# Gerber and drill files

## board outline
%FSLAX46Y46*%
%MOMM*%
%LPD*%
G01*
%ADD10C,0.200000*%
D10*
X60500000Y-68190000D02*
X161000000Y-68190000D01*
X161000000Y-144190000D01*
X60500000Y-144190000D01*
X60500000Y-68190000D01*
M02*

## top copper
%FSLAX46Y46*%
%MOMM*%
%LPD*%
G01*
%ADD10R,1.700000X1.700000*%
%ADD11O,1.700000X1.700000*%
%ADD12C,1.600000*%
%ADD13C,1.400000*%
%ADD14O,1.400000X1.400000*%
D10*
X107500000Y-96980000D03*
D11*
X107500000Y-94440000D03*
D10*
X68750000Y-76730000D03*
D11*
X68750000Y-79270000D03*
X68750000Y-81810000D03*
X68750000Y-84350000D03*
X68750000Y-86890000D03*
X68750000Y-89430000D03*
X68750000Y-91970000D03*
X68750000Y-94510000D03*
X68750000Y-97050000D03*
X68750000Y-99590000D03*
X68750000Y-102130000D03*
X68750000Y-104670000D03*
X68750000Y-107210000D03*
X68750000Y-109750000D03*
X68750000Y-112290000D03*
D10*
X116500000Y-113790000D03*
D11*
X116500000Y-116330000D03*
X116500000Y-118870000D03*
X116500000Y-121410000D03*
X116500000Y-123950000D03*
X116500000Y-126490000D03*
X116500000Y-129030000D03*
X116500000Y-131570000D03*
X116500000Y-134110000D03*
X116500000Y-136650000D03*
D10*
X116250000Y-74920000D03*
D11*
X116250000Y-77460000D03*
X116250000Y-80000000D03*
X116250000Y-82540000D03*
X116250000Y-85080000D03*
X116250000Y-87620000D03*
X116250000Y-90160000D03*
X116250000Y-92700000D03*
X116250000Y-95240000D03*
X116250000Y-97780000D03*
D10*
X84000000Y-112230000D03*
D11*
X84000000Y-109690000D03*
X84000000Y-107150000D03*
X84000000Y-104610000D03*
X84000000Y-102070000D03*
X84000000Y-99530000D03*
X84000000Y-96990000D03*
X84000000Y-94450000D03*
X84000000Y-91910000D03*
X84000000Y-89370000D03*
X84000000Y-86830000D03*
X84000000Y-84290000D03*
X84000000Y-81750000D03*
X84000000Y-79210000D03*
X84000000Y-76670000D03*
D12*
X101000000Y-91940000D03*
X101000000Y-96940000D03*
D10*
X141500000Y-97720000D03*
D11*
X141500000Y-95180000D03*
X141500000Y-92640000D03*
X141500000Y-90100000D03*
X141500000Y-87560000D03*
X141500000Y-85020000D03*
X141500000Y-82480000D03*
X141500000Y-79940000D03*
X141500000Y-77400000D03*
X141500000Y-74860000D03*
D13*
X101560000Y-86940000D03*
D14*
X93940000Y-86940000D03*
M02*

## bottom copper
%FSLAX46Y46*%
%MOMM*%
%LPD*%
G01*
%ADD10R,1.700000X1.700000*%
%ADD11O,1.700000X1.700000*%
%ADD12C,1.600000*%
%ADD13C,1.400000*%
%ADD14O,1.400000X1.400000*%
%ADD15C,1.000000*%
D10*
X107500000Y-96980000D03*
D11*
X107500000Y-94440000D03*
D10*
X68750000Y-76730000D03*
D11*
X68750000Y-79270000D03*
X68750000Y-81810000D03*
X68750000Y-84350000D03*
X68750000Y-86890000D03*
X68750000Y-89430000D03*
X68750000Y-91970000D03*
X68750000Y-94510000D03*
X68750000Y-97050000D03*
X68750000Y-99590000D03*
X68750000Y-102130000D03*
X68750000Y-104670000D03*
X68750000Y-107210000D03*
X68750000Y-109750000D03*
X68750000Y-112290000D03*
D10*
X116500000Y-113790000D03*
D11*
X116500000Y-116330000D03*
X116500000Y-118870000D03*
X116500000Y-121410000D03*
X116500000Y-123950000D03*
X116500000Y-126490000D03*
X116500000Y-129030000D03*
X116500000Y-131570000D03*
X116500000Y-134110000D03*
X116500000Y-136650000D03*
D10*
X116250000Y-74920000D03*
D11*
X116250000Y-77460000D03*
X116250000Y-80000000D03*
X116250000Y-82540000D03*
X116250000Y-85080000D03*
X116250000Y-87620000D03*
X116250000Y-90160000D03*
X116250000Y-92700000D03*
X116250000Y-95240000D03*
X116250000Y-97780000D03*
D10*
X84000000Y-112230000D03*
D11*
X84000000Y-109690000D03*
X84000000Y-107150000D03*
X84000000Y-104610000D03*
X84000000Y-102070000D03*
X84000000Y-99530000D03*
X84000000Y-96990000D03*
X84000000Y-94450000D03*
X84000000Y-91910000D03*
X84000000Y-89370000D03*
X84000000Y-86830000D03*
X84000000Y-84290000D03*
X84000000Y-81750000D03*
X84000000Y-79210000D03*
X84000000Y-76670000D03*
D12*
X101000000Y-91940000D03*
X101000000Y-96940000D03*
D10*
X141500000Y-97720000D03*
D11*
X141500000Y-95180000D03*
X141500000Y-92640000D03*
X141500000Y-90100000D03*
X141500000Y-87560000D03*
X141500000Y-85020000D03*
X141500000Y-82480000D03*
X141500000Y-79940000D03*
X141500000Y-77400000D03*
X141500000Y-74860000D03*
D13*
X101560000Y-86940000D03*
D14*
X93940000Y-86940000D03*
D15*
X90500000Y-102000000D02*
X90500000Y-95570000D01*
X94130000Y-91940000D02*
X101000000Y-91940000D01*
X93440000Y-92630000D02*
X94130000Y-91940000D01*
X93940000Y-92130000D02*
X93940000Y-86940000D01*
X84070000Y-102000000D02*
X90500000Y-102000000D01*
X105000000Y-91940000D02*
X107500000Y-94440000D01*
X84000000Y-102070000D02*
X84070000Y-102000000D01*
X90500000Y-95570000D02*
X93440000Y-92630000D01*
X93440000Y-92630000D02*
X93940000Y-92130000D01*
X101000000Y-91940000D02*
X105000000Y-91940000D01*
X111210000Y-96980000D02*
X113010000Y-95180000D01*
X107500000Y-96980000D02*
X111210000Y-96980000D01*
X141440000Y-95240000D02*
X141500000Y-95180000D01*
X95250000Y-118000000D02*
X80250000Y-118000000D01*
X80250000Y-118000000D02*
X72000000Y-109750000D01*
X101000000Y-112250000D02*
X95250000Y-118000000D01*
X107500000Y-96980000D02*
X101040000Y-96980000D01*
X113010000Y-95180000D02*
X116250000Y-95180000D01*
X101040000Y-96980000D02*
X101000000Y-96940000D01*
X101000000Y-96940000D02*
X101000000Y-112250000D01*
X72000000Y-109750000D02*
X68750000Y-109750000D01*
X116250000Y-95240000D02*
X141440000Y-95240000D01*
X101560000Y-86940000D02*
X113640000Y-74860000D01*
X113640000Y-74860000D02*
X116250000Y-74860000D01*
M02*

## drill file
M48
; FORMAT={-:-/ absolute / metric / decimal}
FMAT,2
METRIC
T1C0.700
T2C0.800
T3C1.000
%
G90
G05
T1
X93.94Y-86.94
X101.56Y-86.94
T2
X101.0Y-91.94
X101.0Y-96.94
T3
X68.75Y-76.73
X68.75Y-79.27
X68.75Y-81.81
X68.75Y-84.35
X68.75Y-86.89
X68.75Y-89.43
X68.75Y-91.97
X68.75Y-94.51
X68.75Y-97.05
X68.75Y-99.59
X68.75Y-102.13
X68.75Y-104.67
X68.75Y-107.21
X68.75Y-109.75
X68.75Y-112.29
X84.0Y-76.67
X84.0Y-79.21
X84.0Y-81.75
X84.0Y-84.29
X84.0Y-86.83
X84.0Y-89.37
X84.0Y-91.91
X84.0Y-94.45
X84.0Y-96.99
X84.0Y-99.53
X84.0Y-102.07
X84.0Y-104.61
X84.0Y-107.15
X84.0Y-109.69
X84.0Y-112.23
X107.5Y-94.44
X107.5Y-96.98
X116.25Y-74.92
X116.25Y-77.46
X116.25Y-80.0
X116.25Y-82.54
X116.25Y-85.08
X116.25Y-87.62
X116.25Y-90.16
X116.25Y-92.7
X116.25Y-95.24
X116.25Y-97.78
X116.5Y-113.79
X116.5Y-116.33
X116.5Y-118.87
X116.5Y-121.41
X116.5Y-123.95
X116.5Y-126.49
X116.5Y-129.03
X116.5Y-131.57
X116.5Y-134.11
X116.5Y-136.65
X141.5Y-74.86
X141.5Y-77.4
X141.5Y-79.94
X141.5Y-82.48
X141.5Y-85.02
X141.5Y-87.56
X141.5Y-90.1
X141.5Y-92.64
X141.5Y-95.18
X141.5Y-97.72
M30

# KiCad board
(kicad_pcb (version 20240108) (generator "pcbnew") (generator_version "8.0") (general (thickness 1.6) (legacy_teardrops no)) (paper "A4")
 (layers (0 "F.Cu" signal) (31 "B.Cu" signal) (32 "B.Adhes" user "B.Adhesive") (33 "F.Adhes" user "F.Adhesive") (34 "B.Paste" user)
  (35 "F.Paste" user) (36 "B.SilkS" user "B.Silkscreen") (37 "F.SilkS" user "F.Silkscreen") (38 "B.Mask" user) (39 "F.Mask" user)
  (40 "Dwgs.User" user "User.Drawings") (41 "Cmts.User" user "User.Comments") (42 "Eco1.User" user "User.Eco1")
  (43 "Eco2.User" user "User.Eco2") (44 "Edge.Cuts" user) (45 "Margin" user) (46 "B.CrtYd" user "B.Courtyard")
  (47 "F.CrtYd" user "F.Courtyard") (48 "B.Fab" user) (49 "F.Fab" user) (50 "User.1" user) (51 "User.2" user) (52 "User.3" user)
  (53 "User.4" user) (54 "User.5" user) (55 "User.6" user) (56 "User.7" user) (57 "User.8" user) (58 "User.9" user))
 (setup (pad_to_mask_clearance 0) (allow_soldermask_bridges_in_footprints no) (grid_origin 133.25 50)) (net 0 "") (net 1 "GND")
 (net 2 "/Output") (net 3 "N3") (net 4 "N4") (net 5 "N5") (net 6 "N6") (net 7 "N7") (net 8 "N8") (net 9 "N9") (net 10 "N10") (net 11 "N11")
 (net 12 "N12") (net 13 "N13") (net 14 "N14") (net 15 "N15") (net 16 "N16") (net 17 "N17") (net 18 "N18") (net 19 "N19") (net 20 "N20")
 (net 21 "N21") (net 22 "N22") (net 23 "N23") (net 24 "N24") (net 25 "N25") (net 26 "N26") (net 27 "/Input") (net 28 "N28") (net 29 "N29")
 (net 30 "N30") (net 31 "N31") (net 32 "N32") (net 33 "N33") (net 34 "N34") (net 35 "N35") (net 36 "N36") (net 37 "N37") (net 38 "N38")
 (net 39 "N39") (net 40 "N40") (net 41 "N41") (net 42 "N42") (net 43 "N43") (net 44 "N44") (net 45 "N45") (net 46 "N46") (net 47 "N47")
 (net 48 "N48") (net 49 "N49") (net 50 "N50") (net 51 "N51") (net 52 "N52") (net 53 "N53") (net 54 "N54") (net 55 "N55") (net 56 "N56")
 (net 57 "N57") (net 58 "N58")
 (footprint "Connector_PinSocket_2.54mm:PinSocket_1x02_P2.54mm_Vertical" (layer "F.Cu") (at 107.5 96.98 180)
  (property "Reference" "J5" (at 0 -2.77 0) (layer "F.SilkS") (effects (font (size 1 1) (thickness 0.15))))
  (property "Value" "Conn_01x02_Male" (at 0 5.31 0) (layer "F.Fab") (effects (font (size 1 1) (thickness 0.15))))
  (pad "1" thru_hole rect (at 0 0 180) (size 1.7 1.7) (drill 1) (layers "*.Cu" "*.Mask") (remove_unused_layers no) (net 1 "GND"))
  (pad "2" thru_hole oval (at 0 2.54 180) (size 1.7 1.7) (drill 1) (layers "*.Cu" "*.Mask") (remove_unused_layers no) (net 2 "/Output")))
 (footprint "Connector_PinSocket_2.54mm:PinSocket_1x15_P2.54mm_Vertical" (layer "F.Cu") (at 68.75 76.73)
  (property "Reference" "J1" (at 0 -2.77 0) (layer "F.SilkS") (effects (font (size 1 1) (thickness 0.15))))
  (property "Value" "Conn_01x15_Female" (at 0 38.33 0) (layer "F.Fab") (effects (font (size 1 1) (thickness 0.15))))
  (pad "1" thru_hole rect (at 0 0) (size 1.7 1.7) (drill 1) (layers "*.Cu" "*.Mask") (remove_unused_layers no) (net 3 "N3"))
  (pad "2" thru_hole oval (at 0 2.54) (size 1.7 1.7) (drill 1) (layers "*.Cu" "*.Mask") (remove_unused_layers no) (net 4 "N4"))
  (pad "3" thru_hole oval (at 0 5.08) (size 1.7 1.7) (drill 1) (layers "*.Cu" "*.Mask") (remove_unused_layers no) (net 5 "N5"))
  (pad "4" thru_hole oval (at 0 7.62) (size 1.7 1.7) (drill 1) (layers "*.Cu" "*.Mask") (remove_unused_layers no) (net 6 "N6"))
  (pad "5" thru_hole oval (at 0 10.16) (size 1.7 1.7) (drill 1) (layers "*.Cu" "*.Mask") (remove_unused_layers no) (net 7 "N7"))
  (pad "6" thru_hole oval (at 0 12.7) (size 1.7 1.7) (drill 1) (layers "*.Cu" "*.Mask") (remove_unused_layers no) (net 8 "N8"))
  (pad "7" thru_hole oval (at 0 15.24) (size 1.7 1.7) (drill 1) (layers "*.Cu" "*.Mask") (remove_unused_layers no) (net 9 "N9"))
  (pad "8" thru_hole oval (at 0 17.78) (size 1.7 1.7) (drill 1) (layers "*.Cu" "*.Mask") (remove_unused_layers no) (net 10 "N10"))
  (pad "9" thru_hole oval (at 0 20.32) (size 1.7 1.7) (drill 1) (layers "*.Cu" "*.Mask") (remove_unused_layers no) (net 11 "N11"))
  (pad "10" thru_hole oval (at 0 22.86) (size 1.7 1.7) (drill 1) (layers "*.Cu" "*.Mask") (remove_unused_layers no) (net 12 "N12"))
  (pad "11" thru_hole oval (at 0 25.4) (size 1.7 1.7) (drill 1) (layers "*.Cu" "*.Mask") (remove_unused_layers no) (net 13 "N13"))
  (pad "12" thru_hole oval (at 0 27.94) (size 1.7 1.7) (drill 1) (layers "*.Cu" "*.Mask") (remove_unused_layers no) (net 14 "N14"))
  (pad "13" thru_hole oval (at 0 30.48) (size 1.7 1.7) (drill 1) (layers "*.Cu" "*.Mask") (remove_unused_layers no) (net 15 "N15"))
  (pad "14" thru_hole oval (at 0 33.02) (size 1.7 1.7) (drill 1) (layers "*.Cu" "*.Mask") (remove_unused_layers no) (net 1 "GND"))
  (pad "15" thru_hole oval (at 0 35.56) (size 1.7 1.7) (drill 1) (layers "*.Cu" "*.Mask") (remove_unused_layers no) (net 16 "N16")))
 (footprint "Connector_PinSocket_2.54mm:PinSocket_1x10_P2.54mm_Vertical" (layer "F.Cu") (at 116.5 113.79)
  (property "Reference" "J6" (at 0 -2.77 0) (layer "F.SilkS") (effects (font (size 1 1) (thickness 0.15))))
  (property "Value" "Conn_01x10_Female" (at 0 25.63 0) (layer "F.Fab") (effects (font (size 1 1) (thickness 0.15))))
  (pad "1" thru_hole rect (at 0 0) (size 1.7 1.7) (drill 1) (layers "*.Cu" "*.Mask") (remove_unused_layers no) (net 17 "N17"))
  (pad "2" thru_hole oval (at 0 2.54) (size 1.7 1.7) (drill 1) (layers "*.Cu" "*.Mask") (remove_unused_layers no) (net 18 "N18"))
  (pad "3" thru_hole oval (at 0 5.08) (size 1.7 1.7) (drill 1) (layers "*.Cu" "*.Mask") (remove_unused_layers no) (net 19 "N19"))
  (pad "4" thru_hole oval (at 0 7.62) (size 1.7 1.7) (drill 1) (layers "*.Cu" "*.Mask") (remove_unused_layers no) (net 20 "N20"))
  (pad "5" thru_hole oval (at 0 10.16) (size 1.7 1.7) (drill 1) (layers "*.Cu" "*.Mask") (remove_unused_layers no) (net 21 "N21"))
  (pad "6" thru_hole oval (at 0 12.7) (size 1.7 1.7) (drill 1) (layers "*.Cu" "*.Mask") (remove_unused_layers no) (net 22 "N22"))
  (pad "7" thru_hole oval (at 0 15.24) (size 1.7 1.7) (drill 1) (layers "*.Cu" "*.Mask") (remove_unused_layers no) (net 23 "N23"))
  (pad "8" thru_hole oval (at 0 17.78) (size 1.7 1.7) (drill 1) (layers "*.Cu" "*.Mask") (remove_unused_layers no) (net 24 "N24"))
  (pad "9" thru_hole oval (at 0 20.32) (size 1.7 1.7) (drill 1) (layers "*.Cu" "*.Mask") (remove_unused_layers no) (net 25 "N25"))
  (pad "10" thru_hole oval (at 0 22.86) (size 1.7 1.7) (drill 1) (layers "*.Cu" "*.Mask") (remove_unused_layers no) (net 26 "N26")))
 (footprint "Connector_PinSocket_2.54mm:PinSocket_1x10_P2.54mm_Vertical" (layer "F.Cu") (at 116.25 74.92)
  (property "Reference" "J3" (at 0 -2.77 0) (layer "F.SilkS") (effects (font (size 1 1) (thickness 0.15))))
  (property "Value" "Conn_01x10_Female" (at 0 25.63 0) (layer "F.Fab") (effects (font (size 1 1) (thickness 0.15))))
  (pad "1" thru_hole rect (at 0 0) (size 1.7 1.7) (drill 1) (layers "*.Cu" "*.Mask") (remove_unused_layers no) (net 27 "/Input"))
  (pad "2" thru_hole oval (at 0 2.54) (size 1.7 1.7) (drill 1) (layers "*.Cu" "*.Mask") (remove_unused_layers no) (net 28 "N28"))
  (pad "3" thru_hole oval (at 0 5.08) (size 1.7 1.7) (drill 1) (layers "*.Cu" "*.Mask") (remove_unused_layers no) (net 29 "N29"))
  (pad "4" thru_hole oval (at 0 7.62) (size 1.7 1.7) (drill 1) (layers "*.Cu" "*.Mask") (remove_unused_layers no) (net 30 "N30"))
  (pad "5" thru_hole oval (at 0 10.16) (size 1.7 1.7) (drill 1) (layers "*.Cu" "*.Mask") (remove_unused_layers no) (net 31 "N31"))
  (pad "6" thru_hole oval (at 0 12.7) (size 1.7 1.7) (drill 1) (layers "*.Cu" "*.Mask") (remove_unused_layers no) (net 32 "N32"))
  (pad "7" thru_hole oval (at 0 15.24) (size 1.7 1.7) (drill 1) (layers "*.Cu" "*.Mask") (remove_unused_layers no) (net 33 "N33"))
  (pad "8" thru_hole oval (at 0 17.78) (size 1.7 1.7) (drill 1) (layers "*.Cu" "*.Mask") (remove_unused_layers no) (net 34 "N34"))
  (pad "9" thru_hole oval (at 0 20.32) (size 1.7 1.7) (drill 1) (layers "*.Cu" "*.Mask") (remove_unused_layers no) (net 1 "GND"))
  (pad "10" thru_hole oval (at 0 22.86) (size 1.7 1.7) (drill 1) (layers "*.Cu" "*.Mask") (remove_unused_layers no) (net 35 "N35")))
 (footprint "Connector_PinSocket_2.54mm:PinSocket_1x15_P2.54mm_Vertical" (layer "F.Cu") (at 84 112.23 180)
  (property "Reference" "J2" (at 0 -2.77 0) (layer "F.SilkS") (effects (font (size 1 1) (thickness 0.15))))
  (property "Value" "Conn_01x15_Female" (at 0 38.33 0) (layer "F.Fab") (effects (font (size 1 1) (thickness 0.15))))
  (pad "1" thru_hole rect (at 0 0 180) (size 1.7 1.7) (drill 1) (layers "*.Cu" "*.Mask") (remove_unused_layers no) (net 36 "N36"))
  (pad "2" thru_hole oval (at 0 2.54 180) (size 1.7 1.7) (drill 1) (layers "*.Cu" "*.Mask") (remove_unused_layers no) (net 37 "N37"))
  (pad "3" thru_hole oval (at 0 5.08 180) (size 1.7 1.7) (drill 1) (layers "*.Cu" "*.Mask") (remove_unused_layers no) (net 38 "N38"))
  (pad "4" thru_hole oval (at 0 7.62 180) (size 1.7 1.7) (drill 1) (layers "*.Cu" "*.Mask") (remove_unused_layers no) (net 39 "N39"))
  (pad "5" thru_hole oval (at 0 10.16 180) (size 1.7 1.7) (drill 1) (layers "*.Cu" "*.Mask") (remove_unused_layers no) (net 2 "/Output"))
  (pad "6" thru_hole oval (at 0 12.7 180) (size 1.7 1.7) (drill 1) (layers "*.Cu" "*.Mask") (remove_unused_layers no) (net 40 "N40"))
  (pad "7" thru_hole oval (at 0 15.24 180) (size 1.7 1.7) (drill 1) (layers "*.Cu" "*.Mask") (remove_unused_layers no) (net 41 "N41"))
  (pad "8" thru_hole oval (at 0 17.78 180) (size 1.7 1.7) (drill 1) (layers "*.Cu" "*.Mask") (remove_unused_layers no) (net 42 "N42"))
  (pad "9" thru_hole oval (at 0 20.32 180) (size 1.7 1.7) (drill 1) (layers "*.Cu" "*.Mask") (remove_unused_layers no) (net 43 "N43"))
  (pad "10" thru_hole oval (at 0 22.86 180) (size 1.7 1.7) (drill 1) (layers "*.Cu" "*.Mask") (remove_unused_layers no) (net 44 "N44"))
  (pad "11" thru_hole oval (at 0 25.4 180) (size 1.7 1.7) (drill 1) (layers "*.Cu" "*.Mask") (remove_unused_layers no) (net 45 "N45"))
  (pad "12" thru_hole oval (at 0 27.94 180) (size 1.7 1.7) (drill 1) (layers "*.Cu" "*.Mask") (remove_unused_layers no) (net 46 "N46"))
  (pad "13" thru_hole oval (at 0 30.48 180) (size 1.7 1.7) (drill 1) (layers "*.Cu" "*.Mask") (remove_unused_layers no) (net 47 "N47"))
  (pad "14" thru_hole oval (at 0 33.02 180) (size 1.7 1.7) (drill 1) (layers "*.Cu" "*.Mask") (remove_unused_layers no) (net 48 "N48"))
  (pad "15" thru_hole oval (at 0 35.56 180) (size 1.7 1.7) (drill 1) (layers "*.Cu" "*.Mask") (remove_unused_layers no) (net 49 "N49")))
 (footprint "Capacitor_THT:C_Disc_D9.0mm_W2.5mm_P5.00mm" (layer "F.Cu") (at 101 91.94 -90)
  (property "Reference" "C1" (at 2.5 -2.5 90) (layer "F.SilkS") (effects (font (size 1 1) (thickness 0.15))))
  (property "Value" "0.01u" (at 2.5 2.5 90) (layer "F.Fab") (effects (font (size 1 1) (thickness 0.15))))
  (pad "1" thru_hole circle (at 0 0 270) (size 1.6 1.6) (drill 0.8) (layers "*.Cu" "*.Mask") (remove_unused_layers no) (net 2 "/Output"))
  (pad "2" thru_hole circle (at 5 0 270) (size 1.6 1.6) (drill 0.8) (layers "*.Cu" "*.Mask") (remove_unused_layers no) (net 1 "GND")))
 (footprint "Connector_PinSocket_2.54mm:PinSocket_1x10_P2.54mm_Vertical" (layer "F.Cu") (at 141.5 97.72 180)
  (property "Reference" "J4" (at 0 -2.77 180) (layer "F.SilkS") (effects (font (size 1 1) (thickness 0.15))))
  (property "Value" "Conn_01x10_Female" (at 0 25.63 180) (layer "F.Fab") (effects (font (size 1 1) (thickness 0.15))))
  (pad "1" thru_hole rect (at 0 0 180) (size 1.7 1.7) (drill 1) (layers "*.Cu" "*.Mask") (remove_unused_layers no) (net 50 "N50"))
  (pad "2" thru_hole oval (at 0 2.54 180) (size 1.7 1.7) (drill 1) (layers "*.Cu" "*.Mask") (remove_unused_layers no) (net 1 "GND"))
  (pad "3" thru_hole oval (at 0 5.08 180) (size 1.7 1.7) (drill 1) (layers "*.Cu" "*.Mask") (remove_unused_layers no) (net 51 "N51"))
  (pad "4" thru_hole oval (at 0 7.62 180) (size 1.7 1.7) (drill 1) (layers "*.Cu" "*.Mask") (remove_unused_layers no) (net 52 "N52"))
  (pad "5" thru_hole oval (at 0 10.16 180) (size 1.7 1.7) (drill 1) (layers "*.Cu" "*.Mask") (remove_unused_layers no) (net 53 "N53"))
  (pad "6" thru_hole oval (at 0 12.7 180) (size 1.7 1.7) (drill 1) (layers "*.Cu" "*.Mask") (remove_unused_layers no) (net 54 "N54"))
  (pad "7" thru_hole oval (at 0 15.24 180) (size 1.7 1.7) (drill 1) (layers "*.Cu" "*.Mask") (remove_unused_layers no) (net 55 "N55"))
  (pad "8" thru_hole oval (at 0 17.78 180) (size 1.7 1.7) (drill 1) (layers "*.Cu" "*.Mask") (remove_unused_layers no) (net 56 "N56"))
  (pad "9" thru_hole oval (at 0 20.32 180) (size 1.7 1.7) (drill 1) (layers "*.Cu" "*.Mask") (remove_unused_layers no) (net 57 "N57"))
  (pad "10" thru_hole oval (at 0 22.86 180) (size 1.7 1.7) (drill 1) (layers "*.Cu" "*.Mask") (remove_unused_layers no) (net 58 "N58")))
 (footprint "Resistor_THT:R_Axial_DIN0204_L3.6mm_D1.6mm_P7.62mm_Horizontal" (layer "F.Cu") (at 101.56 86.94 180)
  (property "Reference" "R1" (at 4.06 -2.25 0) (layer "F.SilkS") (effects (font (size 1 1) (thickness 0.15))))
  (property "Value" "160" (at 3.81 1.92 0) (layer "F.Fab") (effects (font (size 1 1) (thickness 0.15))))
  (pad "1" thru_hole circle (at 0 0 180) (size 1.4 1.4) (drill 0.7) (layers "*.Cu" "*.Mask") (remove_unused_layers no) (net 27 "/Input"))
  (pad "2" thru_hole oval (at 7.62 0 180) (size 1.4 1.4) (drill 0.7) (layers "*.Cu" "*.Mask") (remove_unused_layers no) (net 2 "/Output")))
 (gr_rect (start 60.5 68.19) (end 161 144.19) (stroke (width 0.2) (type default)) (fill none) (layer "Edge.Cuts"))
 (segment (start 90.5 102) (end 90.5 95.57) (width 1) (layer "B.Cu") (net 2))
 (segment (start 94.13 91.94) (end 101 91.94) (width 1) (layer "B.Cu") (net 2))
 (segment (start 93.44 92.63) (end 94.13 91.94) (width 1) (layer "B.Cu") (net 2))
 (segment (start 93.94 92.13) (end 93.94 86.94) (width 1) (layer "B.Cu") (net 2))
 (segment (start 84.07 102) (end 90.5 102) (width 1) (layer "B.Cu") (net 2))
 (segment (start 105 91.94) (end 107.5 94.44) (width 1) (layer "B.Cu") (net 2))
 (segment (start 84 102.07) (end 84.07 102) (width 1) (layer "B.Cu") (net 2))
 (segment (start 90.5 95.57) (end 93.44 92.63) (width 1) (layer "B.Cu") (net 2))
 (segment (start 93.44 92.63) (end 93.94 92.13) (width 1) (layer "B.Cu") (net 2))
 (segment (start 101 91.94) (end 105 91.94) (width 1) (layer "B.Cu") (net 2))
 (segment (start 111.21 96.98) (end 113.01 95.18) (width 1) (layer "B.Cu") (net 1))
 (segment (start 107.5 96.98) (end 111.21 96.98) (width 1) (layer "B.Cu") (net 1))
 (segment (start 141.44 95.24) (end 141.5 95.18) (width 1) (layer "B.Cu") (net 1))
 (segment (start 95.25 118) (end 80.25 118) (width 1) (layer "B.Cu") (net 1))
 (segment (start 80.25 118) (end 72 109.75) (width 1) (layer "B.Cu") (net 1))
 (segment (start 101 112.25) (end 95.25 118) (width 1) (layer "B.Cu") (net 1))
 (segment (start 107.5 96.98) (end 101.04 96.98) (width 1) (layer "B.Cu") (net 1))
 (segment (start 113.01 95.18) (end 116.25 95.18) (width 1) (layer "B.Cu") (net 1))
 (segment (start 101.04 96.98) (end 101 96.94) (width 1) (layer "B.Cu") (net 1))
 (segment (start 101 96.94) (end 101 112.25) (width 1) (layer "B.Cu") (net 1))
 (segment (start 72 109.75) (end 68.75 109.75) (width 1) (layer "B.Cu") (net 1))
 (segment (start 116.25 95.24) (end 141.44 95.24) (width 1) (layer "B.Cu") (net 1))
 (segment (start 101.56 86.94) (end 113.64 74.86) (width 1) (layer "B.Cu") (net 27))
 (segment (start 113.64 74.86) (end 116.25 74.86) (width 1) (layer "B.Cu") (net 27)))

